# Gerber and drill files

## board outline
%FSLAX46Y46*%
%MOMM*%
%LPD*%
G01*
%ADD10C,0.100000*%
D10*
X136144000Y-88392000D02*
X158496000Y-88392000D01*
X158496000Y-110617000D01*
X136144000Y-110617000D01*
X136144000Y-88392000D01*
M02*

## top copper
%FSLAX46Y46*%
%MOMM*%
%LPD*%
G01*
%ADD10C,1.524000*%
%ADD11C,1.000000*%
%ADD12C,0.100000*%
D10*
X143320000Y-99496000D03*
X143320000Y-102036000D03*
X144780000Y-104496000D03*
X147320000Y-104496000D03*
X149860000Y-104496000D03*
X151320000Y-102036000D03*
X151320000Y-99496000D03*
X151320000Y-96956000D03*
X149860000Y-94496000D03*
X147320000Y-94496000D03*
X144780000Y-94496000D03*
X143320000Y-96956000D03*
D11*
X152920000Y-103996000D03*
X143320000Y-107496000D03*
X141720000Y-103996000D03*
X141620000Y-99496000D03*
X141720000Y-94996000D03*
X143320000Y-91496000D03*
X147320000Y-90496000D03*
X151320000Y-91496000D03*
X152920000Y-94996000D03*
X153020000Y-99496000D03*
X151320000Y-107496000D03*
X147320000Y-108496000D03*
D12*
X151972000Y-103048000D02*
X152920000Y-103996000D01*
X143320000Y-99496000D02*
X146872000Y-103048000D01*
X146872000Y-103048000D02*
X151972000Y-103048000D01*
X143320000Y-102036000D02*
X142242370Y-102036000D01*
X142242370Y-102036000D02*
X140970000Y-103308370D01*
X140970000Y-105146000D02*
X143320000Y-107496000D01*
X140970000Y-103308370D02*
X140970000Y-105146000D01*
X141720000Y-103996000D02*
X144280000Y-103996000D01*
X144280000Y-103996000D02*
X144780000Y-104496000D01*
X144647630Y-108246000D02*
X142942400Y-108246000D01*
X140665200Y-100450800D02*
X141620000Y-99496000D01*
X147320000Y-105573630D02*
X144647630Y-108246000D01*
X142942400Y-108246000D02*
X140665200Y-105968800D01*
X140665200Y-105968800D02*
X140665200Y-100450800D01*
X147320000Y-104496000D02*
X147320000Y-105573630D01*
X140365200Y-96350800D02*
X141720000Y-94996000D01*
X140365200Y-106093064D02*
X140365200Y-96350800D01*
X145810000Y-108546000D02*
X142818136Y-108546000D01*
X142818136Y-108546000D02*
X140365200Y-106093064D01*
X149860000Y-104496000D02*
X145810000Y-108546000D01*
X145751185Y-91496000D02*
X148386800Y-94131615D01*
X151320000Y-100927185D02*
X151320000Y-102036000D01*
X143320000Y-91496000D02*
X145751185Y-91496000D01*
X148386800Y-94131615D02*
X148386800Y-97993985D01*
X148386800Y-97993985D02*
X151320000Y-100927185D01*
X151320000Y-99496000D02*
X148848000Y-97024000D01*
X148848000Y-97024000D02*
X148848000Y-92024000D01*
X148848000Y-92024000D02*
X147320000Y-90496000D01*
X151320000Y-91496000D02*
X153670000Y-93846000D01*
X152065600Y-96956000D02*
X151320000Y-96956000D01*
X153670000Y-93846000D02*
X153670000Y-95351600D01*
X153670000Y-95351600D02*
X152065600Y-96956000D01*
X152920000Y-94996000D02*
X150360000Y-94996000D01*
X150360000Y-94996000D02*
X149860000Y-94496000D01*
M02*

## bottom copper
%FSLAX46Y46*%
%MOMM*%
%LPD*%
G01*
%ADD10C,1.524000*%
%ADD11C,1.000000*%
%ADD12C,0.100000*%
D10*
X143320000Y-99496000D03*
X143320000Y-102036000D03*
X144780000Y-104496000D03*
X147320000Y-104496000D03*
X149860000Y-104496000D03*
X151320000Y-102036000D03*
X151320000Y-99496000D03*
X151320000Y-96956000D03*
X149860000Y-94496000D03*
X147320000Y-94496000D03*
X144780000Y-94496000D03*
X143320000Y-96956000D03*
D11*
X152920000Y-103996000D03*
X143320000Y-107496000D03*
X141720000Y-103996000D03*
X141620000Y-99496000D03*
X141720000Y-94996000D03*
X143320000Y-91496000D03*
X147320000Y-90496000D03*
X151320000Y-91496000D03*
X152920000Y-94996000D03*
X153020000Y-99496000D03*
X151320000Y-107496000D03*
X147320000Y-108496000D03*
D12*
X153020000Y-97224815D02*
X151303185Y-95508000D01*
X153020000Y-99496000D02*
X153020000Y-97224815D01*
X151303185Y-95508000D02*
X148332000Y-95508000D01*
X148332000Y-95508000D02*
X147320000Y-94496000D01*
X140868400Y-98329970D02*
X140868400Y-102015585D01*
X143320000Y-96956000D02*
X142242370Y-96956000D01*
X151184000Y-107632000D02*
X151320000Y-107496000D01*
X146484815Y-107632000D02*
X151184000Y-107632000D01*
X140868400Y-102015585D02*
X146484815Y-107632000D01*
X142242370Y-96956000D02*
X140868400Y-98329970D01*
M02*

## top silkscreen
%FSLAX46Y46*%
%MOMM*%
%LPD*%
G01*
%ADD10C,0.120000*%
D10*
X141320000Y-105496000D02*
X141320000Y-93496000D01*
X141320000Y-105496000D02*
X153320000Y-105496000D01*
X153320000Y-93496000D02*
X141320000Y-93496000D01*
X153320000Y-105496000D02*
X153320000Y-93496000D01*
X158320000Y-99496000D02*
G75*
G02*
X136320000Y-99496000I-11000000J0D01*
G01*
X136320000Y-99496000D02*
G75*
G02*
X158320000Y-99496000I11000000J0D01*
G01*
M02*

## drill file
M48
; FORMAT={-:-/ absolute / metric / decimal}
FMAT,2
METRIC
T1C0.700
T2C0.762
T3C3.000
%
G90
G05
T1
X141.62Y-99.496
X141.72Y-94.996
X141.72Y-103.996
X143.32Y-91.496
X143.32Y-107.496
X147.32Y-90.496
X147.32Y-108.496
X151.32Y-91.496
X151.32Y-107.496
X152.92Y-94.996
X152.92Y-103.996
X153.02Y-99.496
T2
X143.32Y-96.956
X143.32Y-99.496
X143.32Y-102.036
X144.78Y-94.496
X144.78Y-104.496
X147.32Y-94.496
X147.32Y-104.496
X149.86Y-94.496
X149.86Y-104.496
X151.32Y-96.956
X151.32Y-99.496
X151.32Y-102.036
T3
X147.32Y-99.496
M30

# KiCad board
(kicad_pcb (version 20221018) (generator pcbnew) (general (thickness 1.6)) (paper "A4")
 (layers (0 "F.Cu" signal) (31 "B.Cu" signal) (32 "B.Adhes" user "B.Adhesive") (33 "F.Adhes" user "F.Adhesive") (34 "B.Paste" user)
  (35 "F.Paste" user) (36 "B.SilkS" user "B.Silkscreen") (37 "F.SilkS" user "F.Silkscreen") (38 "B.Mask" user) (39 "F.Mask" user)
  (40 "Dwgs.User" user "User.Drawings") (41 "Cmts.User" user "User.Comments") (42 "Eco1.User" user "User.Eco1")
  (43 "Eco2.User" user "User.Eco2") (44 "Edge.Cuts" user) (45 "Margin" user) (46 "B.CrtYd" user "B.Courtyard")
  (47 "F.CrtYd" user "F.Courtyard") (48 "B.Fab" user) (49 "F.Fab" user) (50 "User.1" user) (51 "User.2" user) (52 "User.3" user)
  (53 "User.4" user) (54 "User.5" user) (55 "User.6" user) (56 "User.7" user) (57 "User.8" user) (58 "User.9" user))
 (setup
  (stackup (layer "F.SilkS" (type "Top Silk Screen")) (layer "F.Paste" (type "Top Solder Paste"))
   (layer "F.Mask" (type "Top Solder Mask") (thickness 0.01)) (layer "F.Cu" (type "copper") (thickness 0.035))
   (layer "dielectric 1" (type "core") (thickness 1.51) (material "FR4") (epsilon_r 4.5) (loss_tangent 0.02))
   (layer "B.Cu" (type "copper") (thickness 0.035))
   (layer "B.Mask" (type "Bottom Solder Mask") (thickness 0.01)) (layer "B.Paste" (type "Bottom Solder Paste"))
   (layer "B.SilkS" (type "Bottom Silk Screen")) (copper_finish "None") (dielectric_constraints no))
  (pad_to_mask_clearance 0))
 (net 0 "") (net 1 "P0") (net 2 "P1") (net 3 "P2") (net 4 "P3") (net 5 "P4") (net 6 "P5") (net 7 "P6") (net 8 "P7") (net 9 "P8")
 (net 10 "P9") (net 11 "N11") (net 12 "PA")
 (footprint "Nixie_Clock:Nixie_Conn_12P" (layer "F.Cu") (at 147.32 99.496)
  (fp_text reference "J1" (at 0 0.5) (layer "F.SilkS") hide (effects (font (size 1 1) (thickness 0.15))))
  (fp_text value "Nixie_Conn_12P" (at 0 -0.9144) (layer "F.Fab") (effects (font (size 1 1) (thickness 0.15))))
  (fp_line (start -6 6) (end -6 -6) (stroke (width 0.12) (type solid)) (layer "F.SilkS"))
  (fp_line (start -6 6) (end 6 6) (stroke (width 0.12) (type solid)) (layer "F.SilkS"))
  (fp_line (start 6 -6) (end -6 -6) (stroke (width 0.12) (type solid)) (layer "F.SilkS"))
  (fp_line (start 6 6) (end 6 -6) (stroke (width 0.12) (type solid)) (layer "F.SilkS"))
  (pad "0" thru_hole circle (at -4 0) (size 1.524 1.524) (drill 0.762) (layers "*.Cu" "*.Mask") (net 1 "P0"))
  (pad "1" thru_hole circle (at -4 2.54) (size 1.524 1.524) (drill 0.762) (layers "*.Cu" "*.Mask") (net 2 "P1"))
  (pad "2" thru_hole circle (at -2.54 5) (size 1.524 1.524) (drill 0.762) (layers "*.Cu" "*.Mask") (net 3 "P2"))
  (pad "3" thru_hole circle (at 0 5) (size 1.524 1.524) (drill 0.762) (layers "*.Cu" "*.Mask") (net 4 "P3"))
  (pad "4" thru_hole circle (at 2.54 5) (size 1.524 1.524) (drill 0.762) (layers "*.Cu" "*.Mask") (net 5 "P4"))
  (pad "5" thru_hole circle (at 4 2.54) (size 1.524 1.524) (drill 0.762) (layers "*.Cu" "*.Mask") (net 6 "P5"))
  (pad "6" thru_hole circle (at 4 0) (size 1.524 1.524) (drill 0.762) (layers "*.Cu" "*.Mask") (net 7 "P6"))
  (pad "7" thru_hole circle (at 4 -2.54) (size 1.524 1.524) (drill 0.762) (layers "*.Cu" "*.Mask") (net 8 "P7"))
  (pad "8" thru_hole circle (at 2.54 -5) (size 1.524 1.524) (drill 0.762) (layers "*.Cu" "*.Mask") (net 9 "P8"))
  (pad "9" thru_hole circle (at 0 -5) (size 1.524 1.524) (drill 0.762) (layers "*.Cu" "*.Mask") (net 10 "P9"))
  (pad "10" thru_hole circle (at -2.54 -5) (size 1.524 1.524) (drill 0.762) (layers "*.Cu" "*.Mask") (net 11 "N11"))
  (pad "A" thru_hole circle (at -4 -2.54) (size 1.524 1.524) (drill 0.762) (layers "*.Cu" "*.Mask") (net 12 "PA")))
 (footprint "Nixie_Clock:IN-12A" (layer "F.Cu") (at 147.32 99.496)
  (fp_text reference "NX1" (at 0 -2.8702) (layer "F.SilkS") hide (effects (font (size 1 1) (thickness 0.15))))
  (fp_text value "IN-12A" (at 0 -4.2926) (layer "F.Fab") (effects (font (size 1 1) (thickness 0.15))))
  (fp_circle (center 0 0) (end 11 0) (stroke (width 0.12) (type solid)) (fill none) (layer "F.SilkS"))
  (pad "" np_thru_hole circle (at 0 0) (size 3 3) (drill 3) (layers "*.Cu" "*.Mask"))
  (pad "0" thru_hole circle (at 5.6 4.5) (size 1 1) (drill 0.7) (layers "*.Cu" "*.Mask") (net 1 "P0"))
  (pad "1" thru_hole circle (at -4 8) (size 1 1) (drill 0.7) (layers "*.Cu" "*.Mask") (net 2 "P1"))
  (pad "2" thru_hole circle (at -5.6 4.5) (size 1 1) (drill 0.7) (layers "*.Cu" "*.Mask") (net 3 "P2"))
  (pad "3" thru_hole circle (at -5.7 0) (size 1 1) (drill 0.7) (layers "*.Cu" "*.Mask") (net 4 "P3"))
  (pad "4" thru_hole circle (at -5.6 -4.5) (size 1 1) (drill 0.7) (layers "*.Cu" "*.Mask") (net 5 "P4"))
  (pad "5" thru_hole circle (at -4 -8) (size 1 1) (drill 0.7) (layers "*.Cu" "*.Mask") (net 6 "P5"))
  (pad "6" thru_hole circle (at 0 -9) (size 1 1) (drill 0.7) (layers "*.Cu" "*.Mask") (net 7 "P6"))
  (pad "7" thru_hole circle (at 4 -8) (size 1 1) (drill 0.7) (layers "*.Cu" "*.Mask") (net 8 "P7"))
  (pad "8" thru_hole circle (at 5.6 -4.5) (size 1 1) (drill 0.7) (layers "*.Cu" "*.Mask") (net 9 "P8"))
  (pad "9" thru_hole circle (at 5.7 0) (size 1 1) (drill 0.7) (layers "*.Cu" "*.Mask") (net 10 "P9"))
  (pad "A" thru_hole circle (at 4 8) (size 1 1) (drill 0.7) (layers "*.Cu" "*.Mask") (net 12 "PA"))
  (pad "DP" thru_hole circle (at 0 9) (size 1 1) (drill 0.7) (layers "*.Cu" "*.Mask")))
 (gr_rect (start 136.144 88.392) (end 158.496 110.617) (stroke (width 0.1) (type default)) (fill none) (layer "Edge.Cuts"))
 (segment (start 151.972 103.048) (end 152.92 103.996) (width 0.1) (layer "F.Cu") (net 1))
 (segment (start 143.32 99.496) (end 146.872 103.048) (width 0.1) (layer "F.Cu") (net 1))
 (segment (start 146.872 103.048) (end 151.972 103.048) (width 0.1) (layer "F.Cu") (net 1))
 (segment (start 143.32 102.036) (end 142.24237 102.036) (width 0.1) (layer "F.Cu") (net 2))
 (segment (start 142.24237 102.036) (end 140.97 103.30837) (width 0.1) (layer "F.Cu") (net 2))
 (segment (start 140.97 105.146) (end 143.32 107.496) (width 0.1) (layer "F.Cu") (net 2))
 (segment (start 140.97 103.30837) (end 140.97 105.146) (width 0.1) (layer "F.Cu") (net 2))
 (segment (start 141.72 103.996) (end 144.28 103.996) (width 0.1) (layer "F.Cu") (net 3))
 (segment (start 144.28 103.996) (end 144.78 104.496) (width 0.1) (layer "F.Cu") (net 3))
 (segment (start 144.64763 108.246) (end 142.9424 108.246) (width 0.1) (layer "F.Cu") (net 4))
 (segment (start 140.6652 100.4508) (end 141.62 99.496) (width 0.1) (layer "F.Cu") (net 4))
 (segment (start 147.32 105.57363) (end 144.64763 108.246) (width 0.1) (layer "F.Cu") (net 4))
 (segment (start 142.9424 108.246) (end 140.6652 105.9688) (width 0.1) (layer "F.Cu") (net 4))
 (segment (start 140.6652 105.9688) (end 140.6652 100.4508) (width 0.1) (layer "F.Cu") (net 4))
 (segment (start 147.32 104.496) (end 147.32 105.57363) (width 0.1) (layer "F.Cu") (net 4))
 (segment (start 140.3652 96.3508) (end 141.72 94.996) (width 0.1) (layer "F.Cu") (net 5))
 (segment (start 140.3652 106.093064) (end 140.3652 96.3508) (width 0.1) (layer "F.Cu") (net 5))
 (segment (start 145.81 108.546) (end 142.818136 108.546) (width 0.1) (layer "F.Cu") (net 5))
 (segment (start 142.818136 108.546) (end 140.3652 106.093064) (width 0.1) (layer "F.Cu") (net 5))
 (segment (start 149.86 104.496) (end 145.81 108.546) (width 0.1) (layer "F.Cu") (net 5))
 (segment (start 145.751185 91.496) (end 148.3868 94.131615) (width 0.1) (layer "F.Cu") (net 6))
 (segment (start 151.32 100.927185) (end 151.32 102.036) (width 0.1) (layer "F.Cu") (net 6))
 (segment (start 143.32 91.496) (end 145.751185 91.496) (width 0.1) (layer "F.Cu") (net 6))
 (segment (start 148.3868 94.131615) (end 148.3868 97.993985) (width 0.1) (layer "F.Cu") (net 6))
 (segment (start 148.3868 97.993985) (end 151.32 100.927185) (width 0.1) (layer "F.Cu") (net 6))
 (segment (start 151.32 99.496) (end 148.848 97.024) (width 0.1) (layer "F.Cu") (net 7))
 (segment (start 148.848 97.024) (end 148.848 92.024) (width 0.1) (layer "F.Cu") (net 7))
 (segment (start 148.848 92.024) (end 147.32 90.496) (width 0.1) (layer "F.Cu") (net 7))
 (segment (start 151.32 91.496) (end 153.67 93.846) (width 0.1) (layer "F.Cu") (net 8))
 (segment (start 152.0656 96.956) (end 151.32 96.956) (width 0.1) (layer "F.Cu") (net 8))
 (segment (start 153.67 93.846) (end 153.67 95.3516) (width 0.1) (layer "F.Cu") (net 8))
 (segment (start 153.67 95.3516) (end 152.0656 96.956) (width 0.1) (layer "F.Cu") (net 8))
 (segment (start 152.92 94.996) (end 150.36 94.996) (width 0.1) (layer "F.Cu") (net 9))
 (segment (start 150.36 94.996) (end 149.86 94.496) (width 0.1) (layer "F.Cu") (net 9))
 (segment (start 153.02 97.224815) (end 151.303185 95.508) (width 0.1) (layer "B.Cu") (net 10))
 (segment (start 153.02 99.496) (end 153.02 97.224815) (width 0.1) (layer "B.Cu") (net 10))
 (segment (start 151.303185 95.508) (end 148.332 95.508) (width 0.1) (layer "B.Cu") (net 10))
 (segment (start 148.332 95.508) (end 147.32 94.496) (width 0.1) (layer "B.Cu") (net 10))
 (segment (start 140.8684 98.32997) (end 140.8684 102.015585) (width 0.1) (layer "B.Cu") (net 12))
 (segment (start 143.32 96.956) (end 142.24237 96.956) (width 0.1) (layer "B.Cu") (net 12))
 (segment (start 151.184 107.632) (end 151.32 107.496) (width 0.1) (layer "B.Cu") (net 12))
 (segment (start 146.484815 107.632) (end 151.184 107.632) (width 0.1) (layer "B.Cu") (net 12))
 (segment (start 140.8684 102.015585) (end 146.484815 107.632) (width 0.1) (layer "B.Cu") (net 12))
 (segment (start 142.24237 96.956) (end 140.8684 98.32997) (width 0.1) (layer "B.Cu") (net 12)))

